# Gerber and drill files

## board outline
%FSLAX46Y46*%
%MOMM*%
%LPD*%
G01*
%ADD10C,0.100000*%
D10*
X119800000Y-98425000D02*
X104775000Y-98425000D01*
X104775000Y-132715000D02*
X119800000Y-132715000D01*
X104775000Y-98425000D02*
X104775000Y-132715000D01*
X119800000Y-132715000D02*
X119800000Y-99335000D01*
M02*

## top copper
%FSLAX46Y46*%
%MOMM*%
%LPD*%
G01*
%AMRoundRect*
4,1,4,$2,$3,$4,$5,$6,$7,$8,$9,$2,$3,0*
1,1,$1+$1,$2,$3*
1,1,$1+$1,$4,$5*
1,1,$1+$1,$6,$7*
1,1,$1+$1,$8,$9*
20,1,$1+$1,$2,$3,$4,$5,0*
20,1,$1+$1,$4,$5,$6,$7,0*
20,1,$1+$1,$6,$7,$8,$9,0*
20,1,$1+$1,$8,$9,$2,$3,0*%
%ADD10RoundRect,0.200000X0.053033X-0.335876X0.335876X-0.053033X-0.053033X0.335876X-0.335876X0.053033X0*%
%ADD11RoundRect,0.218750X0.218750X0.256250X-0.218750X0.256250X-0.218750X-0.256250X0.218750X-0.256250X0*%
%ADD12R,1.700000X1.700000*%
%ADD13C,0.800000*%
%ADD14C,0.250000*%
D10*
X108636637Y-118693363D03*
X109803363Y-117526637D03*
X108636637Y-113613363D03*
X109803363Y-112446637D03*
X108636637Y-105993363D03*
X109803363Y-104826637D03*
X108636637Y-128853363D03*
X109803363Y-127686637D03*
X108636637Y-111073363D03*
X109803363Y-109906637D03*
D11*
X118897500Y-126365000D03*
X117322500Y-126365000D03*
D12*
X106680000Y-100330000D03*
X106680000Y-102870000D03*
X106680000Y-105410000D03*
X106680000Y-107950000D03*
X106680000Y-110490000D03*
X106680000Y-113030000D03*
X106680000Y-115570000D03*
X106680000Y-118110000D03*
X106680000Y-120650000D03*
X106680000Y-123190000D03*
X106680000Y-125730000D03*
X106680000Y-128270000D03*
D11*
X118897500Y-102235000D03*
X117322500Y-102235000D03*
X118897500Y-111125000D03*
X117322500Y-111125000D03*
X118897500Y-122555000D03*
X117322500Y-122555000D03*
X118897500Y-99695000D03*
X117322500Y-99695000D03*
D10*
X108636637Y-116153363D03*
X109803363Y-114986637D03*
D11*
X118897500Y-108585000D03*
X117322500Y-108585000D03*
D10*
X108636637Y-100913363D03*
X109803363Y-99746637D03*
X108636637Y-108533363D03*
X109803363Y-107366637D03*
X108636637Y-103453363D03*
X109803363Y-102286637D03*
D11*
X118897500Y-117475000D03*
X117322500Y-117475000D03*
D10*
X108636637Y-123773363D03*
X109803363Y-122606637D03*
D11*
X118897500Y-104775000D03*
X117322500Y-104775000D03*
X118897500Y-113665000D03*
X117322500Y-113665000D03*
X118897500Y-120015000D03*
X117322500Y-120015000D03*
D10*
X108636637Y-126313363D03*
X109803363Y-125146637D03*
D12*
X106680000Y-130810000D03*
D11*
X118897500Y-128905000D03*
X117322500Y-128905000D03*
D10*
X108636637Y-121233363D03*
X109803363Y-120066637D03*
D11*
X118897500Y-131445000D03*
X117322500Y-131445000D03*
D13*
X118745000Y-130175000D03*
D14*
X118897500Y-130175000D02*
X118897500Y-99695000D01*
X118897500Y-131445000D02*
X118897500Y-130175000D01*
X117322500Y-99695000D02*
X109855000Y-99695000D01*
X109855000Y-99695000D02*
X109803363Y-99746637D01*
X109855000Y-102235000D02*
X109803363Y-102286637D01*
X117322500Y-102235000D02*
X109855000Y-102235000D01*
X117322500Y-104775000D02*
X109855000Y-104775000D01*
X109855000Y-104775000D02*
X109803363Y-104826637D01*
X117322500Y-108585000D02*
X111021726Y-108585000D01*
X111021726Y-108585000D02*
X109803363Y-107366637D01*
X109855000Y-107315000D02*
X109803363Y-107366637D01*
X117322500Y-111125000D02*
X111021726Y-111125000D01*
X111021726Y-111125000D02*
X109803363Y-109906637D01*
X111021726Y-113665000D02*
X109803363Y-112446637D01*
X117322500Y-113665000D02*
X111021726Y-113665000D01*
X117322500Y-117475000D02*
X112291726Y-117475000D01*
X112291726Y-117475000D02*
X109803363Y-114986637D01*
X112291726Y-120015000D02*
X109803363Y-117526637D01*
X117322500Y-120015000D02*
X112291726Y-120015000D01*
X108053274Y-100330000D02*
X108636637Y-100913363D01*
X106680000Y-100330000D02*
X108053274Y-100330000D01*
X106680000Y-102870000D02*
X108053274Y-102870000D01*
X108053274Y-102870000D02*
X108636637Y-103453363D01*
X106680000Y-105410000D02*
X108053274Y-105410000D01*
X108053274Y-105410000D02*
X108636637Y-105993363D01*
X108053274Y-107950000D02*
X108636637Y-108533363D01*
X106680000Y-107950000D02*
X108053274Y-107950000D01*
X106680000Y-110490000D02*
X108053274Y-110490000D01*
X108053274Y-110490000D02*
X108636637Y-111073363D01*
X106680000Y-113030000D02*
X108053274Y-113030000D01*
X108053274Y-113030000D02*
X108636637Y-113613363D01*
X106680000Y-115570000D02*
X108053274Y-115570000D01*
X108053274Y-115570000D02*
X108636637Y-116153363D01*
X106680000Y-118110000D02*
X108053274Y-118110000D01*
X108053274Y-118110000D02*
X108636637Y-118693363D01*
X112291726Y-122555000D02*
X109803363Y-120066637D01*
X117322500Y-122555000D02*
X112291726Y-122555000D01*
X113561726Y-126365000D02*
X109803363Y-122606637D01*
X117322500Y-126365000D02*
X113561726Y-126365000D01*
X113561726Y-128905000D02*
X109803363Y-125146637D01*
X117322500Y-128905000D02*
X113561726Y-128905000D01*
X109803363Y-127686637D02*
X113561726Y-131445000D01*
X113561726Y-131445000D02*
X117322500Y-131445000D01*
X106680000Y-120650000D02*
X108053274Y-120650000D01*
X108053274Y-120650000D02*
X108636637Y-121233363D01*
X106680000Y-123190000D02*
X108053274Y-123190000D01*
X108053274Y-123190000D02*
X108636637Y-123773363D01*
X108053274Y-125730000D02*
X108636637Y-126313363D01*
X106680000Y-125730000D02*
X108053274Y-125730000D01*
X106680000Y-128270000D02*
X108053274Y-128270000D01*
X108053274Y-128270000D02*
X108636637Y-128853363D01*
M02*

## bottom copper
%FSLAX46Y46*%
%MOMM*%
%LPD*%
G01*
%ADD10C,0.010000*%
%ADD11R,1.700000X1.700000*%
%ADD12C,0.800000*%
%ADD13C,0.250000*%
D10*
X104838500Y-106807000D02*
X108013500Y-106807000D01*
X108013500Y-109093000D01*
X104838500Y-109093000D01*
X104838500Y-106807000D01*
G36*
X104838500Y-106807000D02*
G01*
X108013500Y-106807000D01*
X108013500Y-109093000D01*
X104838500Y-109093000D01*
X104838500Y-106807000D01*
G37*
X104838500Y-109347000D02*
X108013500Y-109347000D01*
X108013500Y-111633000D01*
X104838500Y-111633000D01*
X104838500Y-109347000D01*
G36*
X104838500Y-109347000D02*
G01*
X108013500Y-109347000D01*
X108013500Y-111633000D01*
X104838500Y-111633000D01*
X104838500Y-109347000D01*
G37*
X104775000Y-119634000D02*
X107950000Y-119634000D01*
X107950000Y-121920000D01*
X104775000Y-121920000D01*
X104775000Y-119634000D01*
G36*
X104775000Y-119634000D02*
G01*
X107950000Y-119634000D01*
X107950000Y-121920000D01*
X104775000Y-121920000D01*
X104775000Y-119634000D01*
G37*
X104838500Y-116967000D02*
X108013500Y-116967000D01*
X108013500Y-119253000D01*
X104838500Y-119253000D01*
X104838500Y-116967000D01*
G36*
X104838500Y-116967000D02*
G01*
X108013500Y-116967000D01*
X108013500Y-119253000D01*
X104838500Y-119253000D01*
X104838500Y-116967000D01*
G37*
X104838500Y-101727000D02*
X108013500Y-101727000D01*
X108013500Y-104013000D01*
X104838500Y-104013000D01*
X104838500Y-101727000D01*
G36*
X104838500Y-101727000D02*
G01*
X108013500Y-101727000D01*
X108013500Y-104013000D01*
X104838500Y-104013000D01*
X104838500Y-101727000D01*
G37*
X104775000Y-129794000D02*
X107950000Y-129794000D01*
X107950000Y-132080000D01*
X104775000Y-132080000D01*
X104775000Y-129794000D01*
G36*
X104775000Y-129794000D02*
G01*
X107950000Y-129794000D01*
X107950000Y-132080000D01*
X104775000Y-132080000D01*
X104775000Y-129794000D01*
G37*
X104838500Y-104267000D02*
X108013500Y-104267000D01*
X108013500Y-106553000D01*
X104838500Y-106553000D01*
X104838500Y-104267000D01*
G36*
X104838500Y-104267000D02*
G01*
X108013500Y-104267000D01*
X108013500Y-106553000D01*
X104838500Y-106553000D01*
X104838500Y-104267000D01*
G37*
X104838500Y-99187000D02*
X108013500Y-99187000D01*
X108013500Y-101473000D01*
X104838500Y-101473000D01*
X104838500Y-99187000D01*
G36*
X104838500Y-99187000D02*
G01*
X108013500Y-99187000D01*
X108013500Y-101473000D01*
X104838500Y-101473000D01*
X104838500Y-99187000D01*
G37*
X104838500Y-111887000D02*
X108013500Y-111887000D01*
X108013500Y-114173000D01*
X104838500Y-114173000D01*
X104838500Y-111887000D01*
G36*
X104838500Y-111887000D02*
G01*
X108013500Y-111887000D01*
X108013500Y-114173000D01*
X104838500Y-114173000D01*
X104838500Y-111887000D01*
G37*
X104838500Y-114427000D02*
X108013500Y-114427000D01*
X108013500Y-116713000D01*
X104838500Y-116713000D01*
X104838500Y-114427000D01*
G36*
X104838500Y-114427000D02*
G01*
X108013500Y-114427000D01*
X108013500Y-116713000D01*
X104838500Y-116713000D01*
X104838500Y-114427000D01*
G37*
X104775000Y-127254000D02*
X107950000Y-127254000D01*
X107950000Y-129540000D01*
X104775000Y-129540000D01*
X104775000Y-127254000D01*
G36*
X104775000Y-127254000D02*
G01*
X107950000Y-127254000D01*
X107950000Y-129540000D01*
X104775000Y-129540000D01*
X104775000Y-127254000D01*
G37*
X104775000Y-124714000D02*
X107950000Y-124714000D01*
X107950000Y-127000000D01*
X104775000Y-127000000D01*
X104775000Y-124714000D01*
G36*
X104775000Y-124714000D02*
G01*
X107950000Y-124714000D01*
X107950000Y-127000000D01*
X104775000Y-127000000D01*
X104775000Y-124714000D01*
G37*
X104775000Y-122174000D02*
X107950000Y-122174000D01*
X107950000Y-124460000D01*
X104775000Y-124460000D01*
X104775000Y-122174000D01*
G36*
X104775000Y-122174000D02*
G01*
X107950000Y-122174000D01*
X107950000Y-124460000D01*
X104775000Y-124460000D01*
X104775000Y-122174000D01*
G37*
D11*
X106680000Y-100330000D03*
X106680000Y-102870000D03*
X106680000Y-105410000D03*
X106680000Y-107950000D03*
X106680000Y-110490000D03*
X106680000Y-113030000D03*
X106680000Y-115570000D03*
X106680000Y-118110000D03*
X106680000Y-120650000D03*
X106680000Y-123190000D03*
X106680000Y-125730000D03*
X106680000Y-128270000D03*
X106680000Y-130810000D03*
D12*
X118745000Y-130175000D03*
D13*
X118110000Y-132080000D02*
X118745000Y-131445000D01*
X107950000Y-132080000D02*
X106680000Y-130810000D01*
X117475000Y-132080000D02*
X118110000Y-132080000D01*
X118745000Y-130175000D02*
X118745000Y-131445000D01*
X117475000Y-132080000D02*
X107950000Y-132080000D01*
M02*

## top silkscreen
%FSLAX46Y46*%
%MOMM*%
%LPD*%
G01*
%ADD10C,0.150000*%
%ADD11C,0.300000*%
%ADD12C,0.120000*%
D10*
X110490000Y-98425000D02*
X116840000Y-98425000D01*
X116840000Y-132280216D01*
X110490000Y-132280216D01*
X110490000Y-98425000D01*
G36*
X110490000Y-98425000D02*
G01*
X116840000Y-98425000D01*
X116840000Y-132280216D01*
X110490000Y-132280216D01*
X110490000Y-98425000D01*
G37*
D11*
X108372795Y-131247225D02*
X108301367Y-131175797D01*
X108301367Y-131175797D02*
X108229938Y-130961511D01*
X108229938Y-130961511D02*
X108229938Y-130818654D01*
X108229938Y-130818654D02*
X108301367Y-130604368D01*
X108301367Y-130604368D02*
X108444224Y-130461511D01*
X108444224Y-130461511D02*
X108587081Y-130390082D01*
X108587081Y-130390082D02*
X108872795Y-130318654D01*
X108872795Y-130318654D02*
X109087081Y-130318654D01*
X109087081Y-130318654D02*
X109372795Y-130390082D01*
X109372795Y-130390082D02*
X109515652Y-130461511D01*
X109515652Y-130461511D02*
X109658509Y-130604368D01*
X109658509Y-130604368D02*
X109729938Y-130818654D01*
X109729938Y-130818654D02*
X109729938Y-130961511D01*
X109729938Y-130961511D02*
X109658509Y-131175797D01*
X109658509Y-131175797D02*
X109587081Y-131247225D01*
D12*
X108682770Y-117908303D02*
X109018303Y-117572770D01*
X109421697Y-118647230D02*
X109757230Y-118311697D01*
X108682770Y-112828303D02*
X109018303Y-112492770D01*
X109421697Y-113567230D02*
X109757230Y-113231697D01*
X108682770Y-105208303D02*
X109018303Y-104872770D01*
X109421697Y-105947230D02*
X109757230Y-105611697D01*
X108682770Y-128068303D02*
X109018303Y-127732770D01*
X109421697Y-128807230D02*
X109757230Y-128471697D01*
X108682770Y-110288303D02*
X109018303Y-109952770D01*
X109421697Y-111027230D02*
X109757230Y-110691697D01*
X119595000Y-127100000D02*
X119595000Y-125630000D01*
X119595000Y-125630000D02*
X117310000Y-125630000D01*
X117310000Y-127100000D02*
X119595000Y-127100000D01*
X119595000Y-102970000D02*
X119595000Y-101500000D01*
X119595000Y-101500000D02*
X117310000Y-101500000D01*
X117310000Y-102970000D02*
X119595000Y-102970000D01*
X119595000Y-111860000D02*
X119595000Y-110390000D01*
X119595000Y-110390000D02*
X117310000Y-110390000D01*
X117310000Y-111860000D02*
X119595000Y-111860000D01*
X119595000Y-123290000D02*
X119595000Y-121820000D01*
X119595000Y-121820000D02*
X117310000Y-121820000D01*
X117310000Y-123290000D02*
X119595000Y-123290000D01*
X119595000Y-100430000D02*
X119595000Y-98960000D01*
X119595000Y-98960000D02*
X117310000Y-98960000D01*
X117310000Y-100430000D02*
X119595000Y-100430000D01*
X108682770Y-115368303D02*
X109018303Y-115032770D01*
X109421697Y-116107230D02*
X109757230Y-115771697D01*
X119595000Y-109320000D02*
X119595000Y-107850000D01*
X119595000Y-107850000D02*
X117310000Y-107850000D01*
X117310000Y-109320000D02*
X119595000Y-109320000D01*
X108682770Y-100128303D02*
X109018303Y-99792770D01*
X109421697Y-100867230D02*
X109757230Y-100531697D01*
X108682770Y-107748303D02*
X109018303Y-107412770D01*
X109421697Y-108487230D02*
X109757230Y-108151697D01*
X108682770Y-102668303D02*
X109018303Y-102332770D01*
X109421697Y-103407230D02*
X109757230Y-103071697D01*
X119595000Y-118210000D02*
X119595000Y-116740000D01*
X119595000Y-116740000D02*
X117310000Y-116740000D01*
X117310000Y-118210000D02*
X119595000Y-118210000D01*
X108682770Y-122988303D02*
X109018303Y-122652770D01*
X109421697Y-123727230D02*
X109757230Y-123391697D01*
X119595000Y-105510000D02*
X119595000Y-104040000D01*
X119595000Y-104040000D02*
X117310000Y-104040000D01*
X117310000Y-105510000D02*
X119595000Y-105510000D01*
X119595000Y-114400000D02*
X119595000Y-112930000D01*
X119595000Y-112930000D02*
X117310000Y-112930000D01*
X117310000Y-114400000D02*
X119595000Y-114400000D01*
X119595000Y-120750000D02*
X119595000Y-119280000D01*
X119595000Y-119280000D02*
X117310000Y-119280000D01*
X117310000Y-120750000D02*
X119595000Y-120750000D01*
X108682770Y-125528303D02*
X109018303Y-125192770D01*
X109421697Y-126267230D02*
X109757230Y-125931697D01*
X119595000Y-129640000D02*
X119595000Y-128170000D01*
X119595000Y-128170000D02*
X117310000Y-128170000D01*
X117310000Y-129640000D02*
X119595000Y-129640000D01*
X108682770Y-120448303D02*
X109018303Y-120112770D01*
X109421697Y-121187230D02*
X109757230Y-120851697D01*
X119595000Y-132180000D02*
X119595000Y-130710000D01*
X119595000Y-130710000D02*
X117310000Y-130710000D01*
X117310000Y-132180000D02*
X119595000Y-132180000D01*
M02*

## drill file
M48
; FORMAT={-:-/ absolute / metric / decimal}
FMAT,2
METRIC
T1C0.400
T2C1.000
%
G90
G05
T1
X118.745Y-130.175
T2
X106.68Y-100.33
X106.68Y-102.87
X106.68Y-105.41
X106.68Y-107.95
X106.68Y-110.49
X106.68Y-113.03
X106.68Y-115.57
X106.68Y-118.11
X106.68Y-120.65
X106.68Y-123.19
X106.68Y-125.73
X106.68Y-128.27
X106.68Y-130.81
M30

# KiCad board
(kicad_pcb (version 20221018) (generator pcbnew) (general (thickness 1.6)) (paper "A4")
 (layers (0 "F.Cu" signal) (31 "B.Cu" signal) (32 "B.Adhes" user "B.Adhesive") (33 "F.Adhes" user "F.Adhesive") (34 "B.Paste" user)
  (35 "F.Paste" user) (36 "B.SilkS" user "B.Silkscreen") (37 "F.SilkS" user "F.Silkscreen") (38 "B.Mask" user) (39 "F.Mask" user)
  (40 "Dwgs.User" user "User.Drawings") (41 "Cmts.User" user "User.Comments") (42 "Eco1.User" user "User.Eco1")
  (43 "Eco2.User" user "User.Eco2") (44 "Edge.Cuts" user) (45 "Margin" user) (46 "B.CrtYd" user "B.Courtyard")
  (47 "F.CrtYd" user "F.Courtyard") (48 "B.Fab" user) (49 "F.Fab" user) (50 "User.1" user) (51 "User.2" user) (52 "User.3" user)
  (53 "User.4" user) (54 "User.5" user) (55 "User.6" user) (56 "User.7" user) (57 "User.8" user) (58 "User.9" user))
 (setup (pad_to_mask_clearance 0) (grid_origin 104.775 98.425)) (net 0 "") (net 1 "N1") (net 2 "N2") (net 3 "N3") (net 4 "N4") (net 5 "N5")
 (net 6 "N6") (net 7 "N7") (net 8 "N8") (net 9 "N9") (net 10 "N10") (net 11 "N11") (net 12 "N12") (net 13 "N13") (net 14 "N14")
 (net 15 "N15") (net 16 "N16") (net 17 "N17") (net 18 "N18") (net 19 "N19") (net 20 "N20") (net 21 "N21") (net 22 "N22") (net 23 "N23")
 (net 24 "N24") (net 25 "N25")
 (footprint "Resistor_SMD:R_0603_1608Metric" (layer "F.Cu") (at 109.22 118.11 45)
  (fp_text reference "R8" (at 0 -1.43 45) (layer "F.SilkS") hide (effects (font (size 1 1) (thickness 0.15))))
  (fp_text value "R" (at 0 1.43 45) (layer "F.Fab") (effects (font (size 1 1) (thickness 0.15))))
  (fp_line (start -0.237258 -0.5225) (end 0.237258 -0.5225) (stroke (width 0.12) (type solid)) (layer "F.SilkS"))
  (fp_line (start -0.237258 0.5225) (end 0.237258 0.5225) (stroke (width 0.12) (type solid)) (layer "F.SilkS"))
  (pad "1" smd roundrect (at -0.825 0 45) (size 0.8 0.95) (layers "F.Cu" "F.Paste" "F.Mask") (roundrect_rratio 0.25) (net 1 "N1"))
  (pad "2" smd roundrect (at 0.825 0 45) (size 0.8 0.95) (layers "F.Cu" "F.Paste" "F.Mask") (roundrect_rratio 0.25) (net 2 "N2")))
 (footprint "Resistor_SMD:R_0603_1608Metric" (layer "F.Cu") (at 109.22 113.03 45)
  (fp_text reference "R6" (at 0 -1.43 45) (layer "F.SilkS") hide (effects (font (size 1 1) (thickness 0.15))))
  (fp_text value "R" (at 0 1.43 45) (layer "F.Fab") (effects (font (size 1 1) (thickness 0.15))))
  (fp_line (start -0.237258 -0.5225) (end 0.237258 -0.5225) (stroke (width 0.12) (type solid)) (layer "F.SilkS"))
  (fp_line (start -0.237258 0.5225) (end 0.237258 0.5225) (stroke (width 0.12) (type solid)) (layer "F.SilkS"))
  (pad "1" smd roundrect (at -0.825 0 45) (size 0.8 0.95) (layers "F.Cu" "F.Paste" "F.Mask") (roundrect_rratio 0.25) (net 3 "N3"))
  (pad "2" smd roundrect (at 0.825 0 45) (size 0.8 0.95) (layers "F.Cu" "F.Paste" "F.Mask") (roundrect_rratio 0.25) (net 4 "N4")))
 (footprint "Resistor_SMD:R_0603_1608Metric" (layer "F.Cu") (at 109.22 105.41 45)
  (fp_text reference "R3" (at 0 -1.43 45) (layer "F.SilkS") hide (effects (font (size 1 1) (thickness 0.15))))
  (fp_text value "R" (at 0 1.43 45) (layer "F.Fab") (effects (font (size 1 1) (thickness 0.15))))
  (fp_line (start -0.237258 -0.5225) (end 0.237258 -0.5225) (stroke (width 0.12) (type solid)) (layer "F.SilkS"))
  (fp_line (start -0.237258 0.5225) (end 0.237258 0.5225) (stroke (width 0.12) (type solid)) (layer "F.SilkS"))
  (pad "1" smd roundrect (at -0.825 0 45) (size 0.8 0.95) (layers "F.Cu" "F.Paste" "F.Mask") (roundrect_rratio 0.25) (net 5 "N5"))
  (pad "2" smd roundrect (at 0.825 0 45) (size 0.8 0.95) (layers "F.Cu" "F.Paste" "F.Mask") (roundrect_rratio 0.25) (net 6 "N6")))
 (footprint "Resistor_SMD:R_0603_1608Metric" (layer "F.Cu") (at 109.22 128.27 45)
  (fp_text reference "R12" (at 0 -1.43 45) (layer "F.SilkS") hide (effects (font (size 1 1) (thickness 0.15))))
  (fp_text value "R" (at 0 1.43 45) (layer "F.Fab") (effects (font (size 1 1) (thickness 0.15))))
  (fp_line (start -0.237258 -0.5225) (end 0.237258 -0.5225) (stroke (width 0.12) (type solid)) (layer "F.SilkS"))
  (fp_line (start -0.237258 0.5225) (end 0.237258 0.5225) (stroke (width 0.12) (type solid)) (layer "F.SilkS"))
  (pad "1" smd roundrect (at -0.825 0 45) (size 0.8 0.95) (layers "F.Cu" "F.Paste" "F.Mask") (roundrect_rratio 0.25) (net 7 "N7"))
  (pad "2" smd roundrect (at 0.825 0 45) (size 0.8 0.95) (layers "F.Cu" "F.Paste" "F.Mask") (roundrect_rratio 0.25) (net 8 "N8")))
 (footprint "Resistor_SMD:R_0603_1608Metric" (layer "F.Cu") (at 109.22 110.49 45)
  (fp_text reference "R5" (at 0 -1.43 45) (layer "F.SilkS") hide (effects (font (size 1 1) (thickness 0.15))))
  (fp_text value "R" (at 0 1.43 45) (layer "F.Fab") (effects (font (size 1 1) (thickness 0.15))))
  (fp_line (start -0.237258 -0.5225) (end 0.237258 -0.5225) (stroke (width 0.12) (type solid)) (layer "F.SilkS"))
  (fp_line (start -0.237258 0.5225) (end 0.237258 0.5225) (stroke (width 0.12) (type solid)) (layer "F.SilkS"))
  (pad "1" smd roundrect (at -0.825 0 45) (size 0.8 0.95) (layers "F.Cu" "F.Paste" "F.Mask") (roundrect_rratio 0.25) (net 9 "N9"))
  (pad "2" smd roundrect (at 0.825 0 45) (size 0.8 0.95) (layers "F.Cu" "F.Paste" "F.Mask") (roundrect_rratio 0.25) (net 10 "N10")))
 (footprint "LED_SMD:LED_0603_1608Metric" (layer "F.Cu") (at 118.11 126.365 180)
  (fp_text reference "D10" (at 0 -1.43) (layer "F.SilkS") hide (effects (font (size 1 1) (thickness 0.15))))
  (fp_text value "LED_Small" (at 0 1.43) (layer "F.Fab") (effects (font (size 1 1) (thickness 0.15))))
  (fp_line (start -1.485 -0.735) (end -1.485 0.735) (stroke (width 0.12) (type solid)) (layer "F.SilkS"))
  (fp_line (start -1.485 0.735) (end 0.8 0.735) (stroke (width 0.12) (type solid)) (layer "F.SilkS"))
  (fp_line (start 0.8 -0.735) (end -1.485 -0.735) (stroke (width 0.12) (type solid)) (layer "F.SilkS"))
  (pad "1" smd roundrect (at -0.7875 0 180) (size 0.875 0.95) (layers "F.Cu" "F.Paste" "F.Mask") (roundrect_rratio 0.25) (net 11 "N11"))
  (pad "2" smd roundrect (at 0.7875 0 180) (size 0.875 0.95) (layers "F.Cu" "F.Paste" "F.Mask") (roundrect_rratio 0.25) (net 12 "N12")))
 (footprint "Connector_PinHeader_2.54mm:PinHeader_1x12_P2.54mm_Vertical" (layer "F.Cu") (at 106.68 100.33)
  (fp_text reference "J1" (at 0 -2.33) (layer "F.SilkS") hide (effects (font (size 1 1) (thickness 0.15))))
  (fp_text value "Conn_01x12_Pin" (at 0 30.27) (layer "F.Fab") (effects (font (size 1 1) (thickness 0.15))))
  (pad "1" thru_hole rect (at 0 0) (size 1.7 1.7) (drill 1) (layers "*.Cu" "*.Mask") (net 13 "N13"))
  (pad "2" thru_hole rect (at 0 2.54) (size 1.7 1.7) (drill 1) (layers "*.Cu" "*.Mask") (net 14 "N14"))
  (pad "3" thru_hole rect (at 0 5.08) (size 1.7 1.7) (drill 1) (layers "*.Cu" "*.Mask") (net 5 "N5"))
  (pad "4" thru_hole rect (at 0 7.62) (size 1.7 1.7) (drill 1) (layers "*.Cu" "*.Mask") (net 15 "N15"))
  (pad "5" thru_hole rect (at 0 10.16) (size 1.7 1.7) (drill 1) (layers "*.Cu" "*.Mask") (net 9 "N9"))
  (pad "6" thru_hole rect (at 0 12.7) (size 1.7 1.7) (drill 1) (layers "*.Cu" "*.Mask") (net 3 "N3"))
  (pad "7" thru_hole rect (at 0 15.24) (size 1.7 1.7) (drill 1) (layers "*.Cu" "*.Mask") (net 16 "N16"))
  (pad "8" thru_hole rect (at 0 17.78) (size 1.7 1.7) (drill 1) (layers "*.Cu" "*.Mask") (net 1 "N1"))
  (pad "9" thru_hole rect (at 0 20.32) (size 1.7 1.7) (drill 1) (layers "*.Cu" "*.Mask") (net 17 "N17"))
  (pad "10" thru_hole rect (at 0 22.86) (size 1.7 1.7) (drill 1) (layers "*.Cu" "*.Mask") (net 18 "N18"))
  (pad "11" thru_hole rect (at 0 25.4) (size 1.7 1.7) (drill 1) (layers "*.Cu" "*.Mask") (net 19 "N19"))
  (pad "12" thru_hole rect (at 0 27.94) (size 1.7 1.7) (drill 1) (layers "*.Cu" "*.Mask") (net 7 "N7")))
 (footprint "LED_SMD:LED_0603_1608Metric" (layer "F.Cu") (at 118.11 102.235 180)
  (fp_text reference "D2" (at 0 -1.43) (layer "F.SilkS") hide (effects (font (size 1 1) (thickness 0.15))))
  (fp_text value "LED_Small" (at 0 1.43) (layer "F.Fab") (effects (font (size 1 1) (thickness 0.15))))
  (fp_line (start -1.485 -0.735) (end -1.485 0.735) (stroke (width 0.12) (type solid)) (layer "F.SilkS"))
  (fp_line (start -1.485 0.735) (end 0.8 0.735) (stroke (width 0.12) (type solid)) (layer "F.SilkS"))
  (fp_line (start 0.8 -0.735) (end -1.485 -0.735) (stroke (width 0.12) (type solid)) (layer "F.SilkS"))
  (pad "1" smd roundrect (at -0.7875 0 180) (size 0.875 0.95) (layers "F.Cu" "F.Paste" "F.Mask") (roundrect_rratio 0.25) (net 11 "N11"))
  (pad "2" smd roundrect (at 0.7875 0 180) (size 0.875 0.95) (layers "F.Cu" "F.Paste" "F.Mask") (roundrect_rratio 0.25) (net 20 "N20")))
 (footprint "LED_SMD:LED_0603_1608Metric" (layer "F.Cu") (at 118.11 111.125 180)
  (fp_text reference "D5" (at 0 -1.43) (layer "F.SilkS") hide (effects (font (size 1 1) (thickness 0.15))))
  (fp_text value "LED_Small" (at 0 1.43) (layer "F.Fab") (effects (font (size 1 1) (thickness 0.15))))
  (fp_line (start -1.485 -0.735) (end -1.485 0.735) (stroke (width 0.12) (type solid)) (layer "F.SilkS"))
  (fp_line (start -1.485 0.735) (end 0.8 0.735) (stroke (width 0.12) (type solid)) (layer "F.SilkS"))
  (fp_line (start 0.8 -0.735) (end -1.485 -0.735) (stroke (width 0.12) (type solid)) (layer "F.SilkS"))
  (pad "1" smd roundrect (at -0.7875 0 180) (size 0.875 0.95) (layers "F.Cu" "F.Paste" "F.Mask") (roundrect_rratio 0.25) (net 11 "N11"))
  (pad "2" smd roundrect (at 0.7875 0 180) (size 0.875 0.95) (layers "F.Cu" "F.Paste" "F.Mask") (roundrect_rratio 0.25) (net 10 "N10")))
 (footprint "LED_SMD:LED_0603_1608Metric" (layer "F.Cu") (at 118.11 122.555 180)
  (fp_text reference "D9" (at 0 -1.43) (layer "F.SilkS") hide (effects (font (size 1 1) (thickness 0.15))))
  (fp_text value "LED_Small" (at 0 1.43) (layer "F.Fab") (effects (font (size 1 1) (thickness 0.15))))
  (fp_line (start -1.485 -0.735) (end -1.485 0.735) (stroke (width 0.12) (type solid)) (layer "F.SilkS"))
  (fp_line (start -1.485 0.735) (end 0.8 0.735) (stroke (width 0.12) (type solid)) (layer "F.SilkS"))
  (fp_line (start 0.8 -0.735) (end -1.485 -0.735) (stroke (width 0.12) (type solid)) (layer "F.SilkS"))
  (pad "1" smd roundrect (at -0.7875 0 180) (size 0.875 0.95) (layers "F.Cu" "F.Paste" "F.Mask") (roundrect_rratio 0.25) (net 11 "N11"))
  (pad "2" smd roundrect (at 0.7875 0 180) (size 0.875 0.95) (layers "F.Cu" "F.Paste" "F.Mask") (roundrect_rratio 0.25) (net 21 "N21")))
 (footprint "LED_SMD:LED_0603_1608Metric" (layer "F.Cu") (at 118.11 99.695 180)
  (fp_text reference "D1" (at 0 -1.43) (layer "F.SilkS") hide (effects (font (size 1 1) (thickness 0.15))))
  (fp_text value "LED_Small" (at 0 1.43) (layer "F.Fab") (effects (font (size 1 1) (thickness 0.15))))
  (fp_line (start -1.485 -0.735) (end -1.485 0.735) (stroke (width 0.12) (type solid)) (layer "F.SilkS"))
  (fp_line (start -1.485 0.735) (end 0.8 0.735) (stroke (width 0.12) (type solid)) (layer "F.SilkS"))
  (fp_line (start 0.8 -0.735) (end -1.485 -0.735) (stroke (width 0.12) (type solid)) (layer "F.SilkS"))
  (pad "1" smd roundrect (at -0.7875 0 180) (size 0.875 0.95) (layers "F.Cu" "F.Paste" "F.Mask") (roundrect_rratio 0.25) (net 11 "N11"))
  (pad "2" smd roundrect (at 0.7875 0 180) (size 0.875 0.95) (layers "F.Cu" "F.Paste" "F.Mask") (roundrect_rratio 0.25) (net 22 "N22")))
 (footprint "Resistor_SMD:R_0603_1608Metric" (layer "F.Cu") (at 109.22 115.57 45)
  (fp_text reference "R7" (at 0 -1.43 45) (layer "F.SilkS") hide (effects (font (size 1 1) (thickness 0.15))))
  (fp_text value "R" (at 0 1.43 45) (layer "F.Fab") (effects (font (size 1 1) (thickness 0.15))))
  (fp_line (start -0.237258 -0.5225) (end 0.237258 -0.5225) (stroke (width 0.12) (type solid)) (layer "F.SilkS"))
  (fp_line (start -0.237258 0.5225) (end 0.237258 0.5225) (stroke (width 0.12) (type solid)) (layer "F.SilkS"))
  (pad "1" smd roundrect (at -0.825 0 45) (size 0.8 0.95) (layers "F.Cu" "F.Paste" "F.Mask") (roundrect_rratio 0.25) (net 16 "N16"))
  (pad "2" smd roundrect (at 0.825 0 45) (size 0.8 0.95) (layers "F.Cu" "F.Paste" "F.Mask") (roundrect_rratio 0.25) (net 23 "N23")))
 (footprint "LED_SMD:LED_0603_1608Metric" (layer "F.Cu") (at 118.11 108.585 180)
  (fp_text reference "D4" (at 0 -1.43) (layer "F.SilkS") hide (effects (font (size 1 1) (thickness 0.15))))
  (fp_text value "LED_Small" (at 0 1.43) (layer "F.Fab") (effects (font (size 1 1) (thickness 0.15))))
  (fp_line (start -1.485 -0.735) (end -1.485 0.735) (stroke (width 0.12) (type solid)) (layer "F.SilkS"))
  (fp_line (start -1.485 0.735) (end 0.8 0.735) (stroke (width 0.12) (type solid)) (layer "F.SilkS"))
  (fp_line (start 0.8 -0.735) (end -1.485 -0.735) (stroke (width 0.12) (type solid)) (layer "F.SilkS"))
  (pad "1" smd roundrect (at -0.7875 0 180) (size 0.875 0.95) (layers "F.Cu" "F.Paste" "F.Mask") (roundrect_rratio 0.25) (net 11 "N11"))
  (pad "2" smd roundrect (at 0.7875 0 180) (size 0.875 0.95) (layers "F.Cu" "F.Paste" "F.Mask") (roundrect_rratio 0.25) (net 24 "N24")))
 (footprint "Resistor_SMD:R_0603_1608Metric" (layer "F.Cu") (at 109.22 100.33 45)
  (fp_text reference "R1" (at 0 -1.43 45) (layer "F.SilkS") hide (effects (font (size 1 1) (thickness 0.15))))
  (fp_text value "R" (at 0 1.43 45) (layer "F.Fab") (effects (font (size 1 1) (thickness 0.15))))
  (fp_line (start -0.237258 -0.5225) (end 0.237258 -0.5225) (stroke (width 0.12) (type solid)) (layer "F.SilkS"))
  (fp_line (start -0.237258 0.5225) (end 0.237258 0.5225) (stroke (width 0.12) (type solid)) (layer "F.SilkS"))
  (pad "1" smd roundrect (at -0.825 0 45) (size 0.8 0.95) (layers "F.Cu" "F.Paste" "F.Mask") (roundrect_rratio 0.25) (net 13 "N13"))
  (pad "2" smd roundrect (at 0.825 0 45) (size 0.8 0.95) (layers "F.Cu" "F.Paste" "F.Mask") (roundrect_rratio 0.25) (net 22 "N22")))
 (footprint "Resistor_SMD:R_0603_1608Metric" (layer "F.Cu") (at 109.22 107.95 45)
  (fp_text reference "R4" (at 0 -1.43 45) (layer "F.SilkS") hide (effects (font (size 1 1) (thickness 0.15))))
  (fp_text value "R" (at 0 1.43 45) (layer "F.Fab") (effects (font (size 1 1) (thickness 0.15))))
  (fp_line (start -0.237258 -0.5225) (end 0.237258 -0.5225) (stroke (width 0.12) (type solid)) (layer "F.SilkS"))
  (fp_line (start -0.237258 0.5225) (end 0.237258 0.5225) (stroke (width 0.12) (type solid)) (layer "F.SilkS"))
  (pad "1" smd roundrect (at -0.825 0 45) (size 0.8 0.95) (layers "F.Cu" "F.Paste" "F.Mask") (roundrect_rratio 0.25) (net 15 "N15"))
  (pad "2" smd roundrect (at 0.825 0 45) (size 0.8 0.95) (layers "F.Cu" "F.Paste" "F.Mask") (roundrect_rratio 0.25) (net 24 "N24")))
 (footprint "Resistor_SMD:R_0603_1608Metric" (layer "F.Cu") (at 109.22 102.87 45)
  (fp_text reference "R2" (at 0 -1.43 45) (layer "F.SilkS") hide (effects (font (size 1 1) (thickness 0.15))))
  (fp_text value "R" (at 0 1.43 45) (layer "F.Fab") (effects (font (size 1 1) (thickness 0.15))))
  (fp_line (start -0.237258 -0.5225) (end 0.237258 -0.5225) (stroke (width 0.12) (type solid)) (layer "F.SilkS"))
  (fp_line (start -0.237258 0.5225) (end 0.237258 0.5225) (stroke (width 0.12) (type solid)) (layer "F.SilkS"))
  (pad "1" smd roundrect (at -0.825 0 45) (size 0.8 0.95) (layers "F.Cu" "F.Paste" "F.Mask") (roundrect_rratio 0.25) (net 14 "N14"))
  (pad "2" smd roundrect (at 0.825 0 45) (size 0.8 0.95) (layers "F.Cu" "F.Paste" "F.Mask") (roundrect_rratio 0.25) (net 20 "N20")))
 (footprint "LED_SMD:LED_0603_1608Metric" (layer "F.Cu") (at 118.11 117.475 180)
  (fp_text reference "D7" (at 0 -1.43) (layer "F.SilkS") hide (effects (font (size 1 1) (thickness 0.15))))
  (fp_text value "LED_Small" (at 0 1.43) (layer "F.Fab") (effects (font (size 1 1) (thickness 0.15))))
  (fp_line (start -1.485 -0.735) (end -1.485 0.735) (stroke (width 0.12) (type solid)) (layer "F.SilkS"))
  (fp_line (start -1.485 0.735) (end 0.8 0.735) (stroke (width 0.12) (type solid)) (layer "F.SilkS"))
  (fp_line (start 0.8 -0.735) (end -1.485 -0.735) (stroke (width 0.12) (type solid)) (layer "F.SilkS"))
  (pad "1" smd roundrect (at -0.7875 0 180) (size 0.875 0.95) (layers "F.Cu" "F.Paste" "F.Mask") (roundrect_rratio 0.25) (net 11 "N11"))
  (pad "2" smd roundrect (at 0.7875 0 180) (size 0.875 0.95) (layers "F.Cu" "F.Paste" "F.Mask") (roundrect_rratio 0.25) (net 23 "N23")))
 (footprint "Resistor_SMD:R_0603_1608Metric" (layer "F.Cu") (at 109.22 123.19 45)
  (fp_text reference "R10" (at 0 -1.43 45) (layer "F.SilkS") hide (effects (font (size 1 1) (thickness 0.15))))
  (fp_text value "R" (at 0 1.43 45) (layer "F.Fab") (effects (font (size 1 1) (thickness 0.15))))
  (fp_line (start -0.237258 -0.5225) (end 0.237258 -0.5225) (stroke (width 0.12) (type solid)) (layer "F.SilkS"))
  (fp_line (start -0.237258 0.5225) (end 0.237258 0.5225) (stroke (width 0.12) (type solid)) (layer "F.SilkS"))
  (pad "1" smd roundrect (at -0.825 0 45) (size 0.8 0.95) (layers "F.Cu" "F.Paste" "F.Mask") (roundrect_rratio 0.25) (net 18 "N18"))
  (pad "2" smd roundrect (at 0.825 0 45) (size 0.8 0.95) (layers "F.Cu" "F.Paste" "F.Mask") (roundrect_rratio 0.25) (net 12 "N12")))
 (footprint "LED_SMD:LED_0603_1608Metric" (layer "F.Cu") (at 118.11 104.775 180)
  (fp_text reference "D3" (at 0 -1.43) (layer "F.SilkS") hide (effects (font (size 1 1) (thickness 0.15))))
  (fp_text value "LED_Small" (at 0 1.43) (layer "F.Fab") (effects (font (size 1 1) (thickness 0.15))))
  (fp_line (start -1.485 -0.735) (end -1.485 0.735) (stroke (width 0.12) (type solid)) (layer "F.SilkS"))
  (fp_line (start -1.485 0.735) (end 0.8 0.735) (stroke (width 0.12) (type solid)) (layer "F.SilkS"))
  (fp_line (start 0.8 -0.735) (end -1.485 -0.735) (stroke (width 0.12) (type solid)) (layer "F.SilkS"))
  (pad "1" smd roundrect (at -0.7875 0 180) (size 0.875 0.95) (layers "F.Cu" "F.Paste" "F.Mask") (roundrect_rratio 0.25) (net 11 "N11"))
  (pad "2" smd roundrect (at 0.7875 0 180) (size 0.875 0.95) (layers "F.Cu" "F.Paste" "F.Mask") (roundrect_rratio 0.25) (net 6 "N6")))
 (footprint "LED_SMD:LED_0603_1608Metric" (layer "F.Cu") (at 118.11 113.665 180)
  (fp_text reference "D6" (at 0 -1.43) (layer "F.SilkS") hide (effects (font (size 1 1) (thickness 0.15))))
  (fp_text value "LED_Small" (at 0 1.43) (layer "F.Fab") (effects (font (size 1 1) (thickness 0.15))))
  (fp_line (start -1.485 -0.735) (end -1.485 0.735) (stroke (width 0.12) (type solid)) (layer "F.SilkS"))
  (fp_line (start -1.485 0.735) (end 0.8 0.735) (stroke (width 0.12) (type solid)) (layer "F.SilkS"))
  (fp_line (start 0.8 -0.735) (end -1.485 -0.735) (stroke (width 0.12) (type solid)) (layer "F.SilkS"))
  (pad "1" smd roundrect (at -0.7875 0 180) (size 0.875 0.95) (layers "F.Cu" "F.Paste" "F.Mask") (roundrect_rratio 0.25) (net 11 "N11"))
  (pad "2" smd roundrect (at 0.7875 0 180) (size 0.875 0.95) (layers "F.Cu" "F.Paste" "F.Mask") (roundrect_rratio 0.25) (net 4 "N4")))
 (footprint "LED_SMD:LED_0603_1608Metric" (layer "F.Cu") (at 118.11 120.015 180)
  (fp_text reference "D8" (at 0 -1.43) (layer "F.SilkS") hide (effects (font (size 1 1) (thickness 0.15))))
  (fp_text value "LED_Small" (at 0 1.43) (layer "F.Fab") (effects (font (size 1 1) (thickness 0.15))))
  (fp_line (start -1.485 -0.735) (end -1.485 0.735) (stroke (width 0.12) (type solid)) (layer "F.SilkS"))
  (fp_line (start -1.485 0.735) (end 0.8 0.735) (stroke (width 0.12) (type solid)) (layer "F.SilkS"))
  (fp_line (start 0.8 -0.735) (end -1.485 -0.735) (stroke (width 0.12) (type solid)) (layer "F.SilkS"))
  (pad "1" smd roundrect (at -0.7875 0 180) (size 0.875 0.95) (layers "F.Cu" "F.Paste" "F.Mask") (roundrect_rratio 0.25) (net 11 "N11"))
  (pad "2" smd roundrect (at 0.7875 0 180) (size 0.875 0.95) (layers "F.Cu" "F.Paste" "F.Mask") (roundrect_rratio 0.25) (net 2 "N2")))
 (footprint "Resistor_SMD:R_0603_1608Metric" (layer "F.Cu") (at 109.22 125.73 45)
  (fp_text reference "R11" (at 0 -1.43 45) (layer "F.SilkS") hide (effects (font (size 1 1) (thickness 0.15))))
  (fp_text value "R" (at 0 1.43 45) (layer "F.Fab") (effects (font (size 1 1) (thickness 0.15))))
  (fp_line (start -0.237258 -0.5225) (end 0.237258 -0.5225) (stroke (width 0.12) (type solid)) (layer "F.SilkS"))
  (fp_line (start -0.237258 0.5225) (end 0.237258 0.5225) (stroke (width 0.12) (type solid)) (layer "F.SilkS"))
  (pad "1" smd roundrect (at -0.825 0 45) (size 0.8 0.95) (layers "F.Cu" "F.Paste" "F.Mask") (roundrect_rratio 0.25) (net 19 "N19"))
  (pad "2" smd roundrect (at 0.825 0 45) (size 0.8 0.95) (layers "F.Cu" "F.Paste" "F.Mask") (roundrect_rratio 0.25) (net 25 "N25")))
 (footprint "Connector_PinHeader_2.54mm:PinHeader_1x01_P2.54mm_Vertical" (layer "F.Cu") (at 106.68 130.81)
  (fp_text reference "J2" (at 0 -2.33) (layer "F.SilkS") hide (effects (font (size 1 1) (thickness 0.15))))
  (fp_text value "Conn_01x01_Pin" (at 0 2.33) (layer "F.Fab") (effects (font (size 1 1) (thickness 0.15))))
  (pad "1" thru_hole rect (at 0 0) (size 1.7 1.7) (drill 1) (layers "*.Cu" "*.Mask") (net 11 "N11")))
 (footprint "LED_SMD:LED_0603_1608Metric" (layer "F.Cu") (at 118.11 128.905 180)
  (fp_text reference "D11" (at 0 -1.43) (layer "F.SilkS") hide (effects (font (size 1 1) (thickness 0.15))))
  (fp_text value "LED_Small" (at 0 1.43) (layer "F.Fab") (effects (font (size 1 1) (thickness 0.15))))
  (fp_line (start -1.485 -0.735) (end -1.485 0.735) (stroke (width 0.12) (type solid)) (layer "F.SilkS"))
  (fp_line (start -1.485 0.735) (end 0.8 0.735) (stroke (width 0.12) (type solid)) (layer "F.SilkS"))
  (fp_line (start 0.8 -0.735) (end -1.485 -0.735) (stroke (width 0.12) (type solid)) (layer "F.SilkS"))
  (pad "1" smd roundrect (at -0.7875 0 180) (size 0.875 0.95) (layers "F.Cu" "F.Paste" "F.Mask") (roundrect_rratio 0.25) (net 11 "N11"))
  (pad "2" smd roundrect (at 0.7875 0 180) (size 0.875 0.95) (layers "F.Cu" "F.Paste" "F.Mask") (roundrect_rratio 0.25) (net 25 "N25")))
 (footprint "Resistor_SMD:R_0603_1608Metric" (layer "F.Cu") (at 109.22 120.65 45)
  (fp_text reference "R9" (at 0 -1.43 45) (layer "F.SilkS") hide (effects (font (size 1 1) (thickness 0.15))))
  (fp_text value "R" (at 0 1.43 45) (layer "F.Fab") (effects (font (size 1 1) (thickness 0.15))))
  (fp_line (start -0.237258 -0.5225) (end 0.237258 -0.5225) (stroke (width 0.12) (type solid)) (layer "F.SilkS"))
  (fp_line (start -0.237258 0.5225) (end 0.237258 0.5225) (stroke (width 0.12) (type solid)) (layer "F.SilkS"))
  (pad "1" smd roundrect (at -0.825 0 45) (size 0.8 0.95) (layers "F.Cu" "F.Paste" "F.Mask") (roundrect_rratio 0.25) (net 17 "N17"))
  (pad "2" smd roundrect (at 0.825 0 45) (size 0.8 0.95) (layers "F.Cu" "F.Paste" "F.Mask") (roundrect_rratio 0.25) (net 21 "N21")))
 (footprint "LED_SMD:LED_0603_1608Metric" (layer "F.Cu") (at 118.11 131.445 180)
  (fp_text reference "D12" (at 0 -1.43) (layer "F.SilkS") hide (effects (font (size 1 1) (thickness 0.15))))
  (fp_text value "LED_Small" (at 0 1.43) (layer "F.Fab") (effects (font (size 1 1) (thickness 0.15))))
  (fp_line (start -1.485 -0.735) (end -1.485 0.735) (stroke (width 0.12) (type solid)) (layer "F.SilkS"))
  (fp_line (start -1.485 0.735) (end 0.8 0.735) (stroke (width 0.12) (type solid)) (layer "F.SilkS"))
  (fp_line (start 0.8 -0.735) (end -1.485 -0.735) (stroke (width 0.12) (type solid)) (layer "F.SilkS"))
  (pad "1" smd roundrect (at -0.7875 0 180) (size 0.875 0.95) (layers "F.Cu" "F.Paste" "F.Mask") (roundrect_rratio 0.25) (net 11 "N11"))
  (pad "2" smd roundrect (at 0.7875 0 180) (size 0.875 0.95) (layers "F.Cu" "F.Paste" "F.Mask") (roundrect_rratio 0.25) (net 8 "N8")))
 (gr_rect (start 104.8385 106.807) (end 108.0135 109.093) (stroke (width 0.01) (type solid)) (fill solid) (layer "B.Cu"))
 (gr_rect (start 104.8385 109.347) (end 108.0135 111.633) (stroke (width 0.01) (type solid)) (fill solid) (layer "B.Cu"))
 (gr_rect (start 104.775 119.634) (end 107.95 121.92) (stroke (width 0.01) (type solid)) (fill solid) (layer "B.Cu"))
 (gr_rect (start 104.8385 116.967) (end 108.0135 119.253) (stroke (width 0.01) (type solid)) (fill solid) (layer "B.Cu"))
 (gr_rect (start 104.8385 101.727) (end 108.0135 104.013) (stroke (width 0.01) (type solid)) (fill solid) (layer "B.Cu"))
 (gr_rect (start 104.775 129.794) (end 107.95 132.08) (stroke (width 0.01) (type solid)) (fill solid) (layer "B.Cu"))
 (gr_rect (start 104.8385 104.267) (end 108.0135 106.553) (stroke (width 0.01) (type solid)) (fill solid) (layer "B.Cu"))
 (gr_rect (start 104.8385 99.187) (end 108.0135 101.473) (stroke (width 0.01) (type solid)) (fill solid) (layer "B.Cu"))
 (gr_rect (start 104.8385 111.887) (end 108.0135 114.173) (stroke (width 0.01) (type solid)) (fill solid) (layer "B.Cu"))
 (gr_rect (start 104.8385 114.427) (end 108.0135 116.713) (stroke (width 0.01) (type solid)) (fill solid) (layer "B.Cu"))
 (gr_rect (start 104.775 127.254) (end 107.95 129.54) (stroke (width 0.01) (type solid)) (fill solid) (layer "B.Cu"))
 (gr_rect (start 104.775 124.714) (end 107.95 127) (stroke (width 0.01) (type solid)) (fill solid) (layer "B.Cu"))
 (gr_rect (start 104.775 122.174) (end 107.95 124.46) (stroke (width 0.01) (type solid)) (fill solid) (layer "B.Cu"))
 (gr_rect (start 110.49 98.425) (end 116.84 132.280216) (stroke (width 0.15) (type solid)) (fill solid) (layer "F.SilkS"))
 (gr_line (start 119.8 98.425) (end 104.775 98.425) (stroke (width 0.1) (type default)) (layer "Edge.Cuts"))
 (gr_line (start 104.775 132.715) (end 119.8 132.715) (stroke (width 0.1) (type default)) (layer "Edge.Cuts"))
 (gr_line (start 104.775 98.425) (end 104.775 132.715) (stroke (width 0.1) (type default)) (layer "Edge.Cuts"))
 (gr_line (start 119.8 132.715) (end 119.8 99.335) (stroke (width 0.1) (type default)) (layer "Edge.Cuts"))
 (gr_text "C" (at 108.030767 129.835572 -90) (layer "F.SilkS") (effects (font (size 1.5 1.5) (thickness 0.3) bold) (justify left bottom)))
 (segment (start 118.8975 130.175) (end 118.8975 99.695) (width 0.25) (layer "F.Cu") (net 11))
 (segment (start 118.8975 131.445) (end 118.8975 130.175) (width 0.25) (layer "F.Cu") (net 11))
 (via (at 118.745 130.175) (size 0.8) (drill 0.4) (layers "F.Cu" "B.Cu") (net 11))
 (segment (start 118.11 132.08) (end 118.745 131.445) (width 0.25) (layer "B.Cu") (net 11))
 (segment (start 107.95 132.08) (end 106.68 130.81) (width 0.25) (layer "B.Cu") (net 11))
 (segment (start 117.475 132.08) (end 118.11 132.08) (width 0.25) (layer "B.Cu") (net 11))
 (segment (start 118.745 130.175) (end 118.745 131.445) (width 0.25) (layer "B.Cu") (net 11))
 (segment (start 117.475 132.08) (end 107.95 132.08) (width 0.25) (layer "B.Cu") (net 11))
 (segment (start 117.3225 99.695) (end 109.855 99.695) (width 0.25) (layer "F.Cu") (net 22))
 (segment (start 109.855 99.695) (end 109.803363 99.746637) (width 0.25) (layer "F.Cu") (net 22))
 (segment (start 109.855 102.235) (end 109.803363 102.286637) (width 0.25) (layer "F.Cu") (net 20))
 (segment (start 117.3225 102.235) (end 109.855 102.235) (width 0.25) (layer "F.Cu") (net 20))
 (segment (start 117.3225 104.775) (end 109.855 104.775) (width 0.25) (layer "F.Cu") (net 6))
 (segment (start 109.855 104.775) (end 109.803363 104.826637) (width 0.25) (layer "F.Cu") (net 6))
 (segment (start 117.3225 108.585) (end 111.021726 108.585) (width 0.25) (layer "F.Cu") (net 24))
 (segment (start 111.021726 108.585) (end 109.803363 107.366637) (width 0.25) (layer "F.Cu") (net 24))
 (segment (start 109.855 107.315) (end 109.803363 107.366637) (width 0.25) (layer "F.Cu") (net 24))
 (segment (start 117.3225 111.125) (end 111.021726 111.125) (width 0.25) (layer "F.Cu") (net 10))
 (segment (start 111.021726 111.125) (end 109.803363 109.906637) (width 0.25) (layer "F.Cu") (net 10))
 (segment (start 111.021726 113.665) (end 109.803363 112.446637) (width 0.25) (layer "F.Cu") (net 4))
 (segment (start 117.3225 113.665) (end 111.021726 113.665) (width 0.25) (layer "F.Cu") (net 4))
 (segment (start 117.3225 117.475) (end 112.291726 117.475) (width 0.25) (layer "F.Cu") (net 23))
 (segment (start 112.291726 117.475) (end 109.803363 114.986637) (width 0.25) (layer "F.Cu") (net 23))
 (segment (start 112.291726 120.015) (end 109.803363 117.526637) (width 0.25) (layer "F.Cu") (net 2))
 (segment (start 117.3225 120.015) (end 112.291726 120.015) (width 0.25) (layer "F.Cu") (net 2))
 (segment (start 108.053274 100.33) (end 108.636637 100.913363) (width 0.25) (layer "F.Cu") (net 13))
 (segment (start 106.68 100.33) (end 108.053274 100.33) (width 0.25) (layer "F.Cu") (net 13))
 (segment (start 106.68 102.87) (end 108.053274 102.87) (width 0.25) (layer "F.Cu") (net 14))
 (segment (start 108.053274 102.87) (end 108.636637 103.453363) (width 0.25) (layer "F.Cu") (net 14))
 (segment (start 106.68 105.41) (end 108.053274 105.41) (width 0.25) (layer "F.Cu") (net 5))
 (segment (start 108.053274 105.41) (end 108.636637 105.993363) (width 0.25) (layer "F.Cu") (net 5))
 (segment (start 108.053274 107.95) (end 108.636637 108.533363) (width 0.25) (layer "F.Cu") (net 15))
 (segment (start 106.68 107.95) (end 108.053274 107.95) (width 0.25) (layer "F.Cu") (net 15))
 (segment (start 106.68 110.49) (end 108.053274 110.49) (width 0.25) (layer "F.Cu") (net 9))
 (segment (start 108.053274 110.49) (end 108.636637 111.073363) (width 0.25) (layer "F.Cu") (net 9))
 (segment (start 106.68 113.03) (end 108.053274 113.03) (width 0.25) (layer "F.Cu") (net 3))
 (segment (start 108.053274 113.03) (end 108.636637 113.613363) (width 0.25) (layer "F.Cu") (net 3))
 (segment (start 106.68 115.57) (end 108.053274 115.57) (width 0.25) (layer "F.Cu") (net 16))
 (segment (start 108.053274 115.57) (end 108.636637 116.153363) (width 0.25) (layer "F.Cu") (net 16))
 (segment (start 106.68 118.11) (end 108.053274 118.11) (width 0.25) (layer "F.Cu") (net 1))
 (segment (start 108.053274 118.11) (end 108.636637 118.693363) (width 0.25) (layer "F.Cu") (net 1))
 (segment (start 112.291726 122.555) (end 109.803363 120.066637) (width 0.25) (layer "F.Cu") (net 21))
 (segment (start 117.3225 122.555) (end 112.291726 122.555) (width 0.25) (layer "F.Cu") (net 21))
 (segment (start 113.561726 126.365) (end 109.803363 122.606637) (width 0.25) (layer "F.Cu") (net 12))
 (segment (start 117.3225 126.365) (end 113.561726 126.365) (width 0.25) (layer "F.Cu") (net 12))
 (segment (start 113.561726 128.905) (end 109.803363 125.146637) (width 0.25) (layer "F.Cu") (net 25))
 (segment (start 117.3225 128.905) (end 113.561726 128.905) (width 0.25) (layer "F.Cu") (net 25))
 (segment (start 109.803363 127.686637) (end 113.561726 131.445) (width 0.25) (layer "F.Cu") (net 8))
 (segment (start 113.561726 131.445) (end 117.3225 131.445) (width 0.25) (layer "F.Cu") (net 8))
 (segment (start 106.68 120.65) (end 108.053274 120.65) (width 0.25) (layer "F.Cu") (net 17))
 (segment (start 108.053274 120.65) (end 108.636637 121.233363) (width 0.25) (layer "F.Cu") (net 17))
 (segment (start 106.68 123.19) (end 108.053274 123.19) (width 0.25) (layer "F.Cu") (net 18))
 (segment (start 108.053274 123.19) (end 108.636637 123.773363) (width 0.25) (layer "F.Cu") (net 18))
 (segment (start 108.053274 125.73) (end 108.636637 126.313363) (width 0.25) (layer "F.Cu") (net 19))
 (segment (start 106.68 125.73) (end 108.053274 125.73) (width 0.25) (layer "F.Cu") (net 19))
 (segment (start 106.68 128.27) (end 108.053274 128.27) (width 0.25) (layer "F.Cu") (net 7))
 (segment (start 108.053274 128.27) (end 108.636637 128.853363) (width 0.25) (layer "F.Cu") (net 7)))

